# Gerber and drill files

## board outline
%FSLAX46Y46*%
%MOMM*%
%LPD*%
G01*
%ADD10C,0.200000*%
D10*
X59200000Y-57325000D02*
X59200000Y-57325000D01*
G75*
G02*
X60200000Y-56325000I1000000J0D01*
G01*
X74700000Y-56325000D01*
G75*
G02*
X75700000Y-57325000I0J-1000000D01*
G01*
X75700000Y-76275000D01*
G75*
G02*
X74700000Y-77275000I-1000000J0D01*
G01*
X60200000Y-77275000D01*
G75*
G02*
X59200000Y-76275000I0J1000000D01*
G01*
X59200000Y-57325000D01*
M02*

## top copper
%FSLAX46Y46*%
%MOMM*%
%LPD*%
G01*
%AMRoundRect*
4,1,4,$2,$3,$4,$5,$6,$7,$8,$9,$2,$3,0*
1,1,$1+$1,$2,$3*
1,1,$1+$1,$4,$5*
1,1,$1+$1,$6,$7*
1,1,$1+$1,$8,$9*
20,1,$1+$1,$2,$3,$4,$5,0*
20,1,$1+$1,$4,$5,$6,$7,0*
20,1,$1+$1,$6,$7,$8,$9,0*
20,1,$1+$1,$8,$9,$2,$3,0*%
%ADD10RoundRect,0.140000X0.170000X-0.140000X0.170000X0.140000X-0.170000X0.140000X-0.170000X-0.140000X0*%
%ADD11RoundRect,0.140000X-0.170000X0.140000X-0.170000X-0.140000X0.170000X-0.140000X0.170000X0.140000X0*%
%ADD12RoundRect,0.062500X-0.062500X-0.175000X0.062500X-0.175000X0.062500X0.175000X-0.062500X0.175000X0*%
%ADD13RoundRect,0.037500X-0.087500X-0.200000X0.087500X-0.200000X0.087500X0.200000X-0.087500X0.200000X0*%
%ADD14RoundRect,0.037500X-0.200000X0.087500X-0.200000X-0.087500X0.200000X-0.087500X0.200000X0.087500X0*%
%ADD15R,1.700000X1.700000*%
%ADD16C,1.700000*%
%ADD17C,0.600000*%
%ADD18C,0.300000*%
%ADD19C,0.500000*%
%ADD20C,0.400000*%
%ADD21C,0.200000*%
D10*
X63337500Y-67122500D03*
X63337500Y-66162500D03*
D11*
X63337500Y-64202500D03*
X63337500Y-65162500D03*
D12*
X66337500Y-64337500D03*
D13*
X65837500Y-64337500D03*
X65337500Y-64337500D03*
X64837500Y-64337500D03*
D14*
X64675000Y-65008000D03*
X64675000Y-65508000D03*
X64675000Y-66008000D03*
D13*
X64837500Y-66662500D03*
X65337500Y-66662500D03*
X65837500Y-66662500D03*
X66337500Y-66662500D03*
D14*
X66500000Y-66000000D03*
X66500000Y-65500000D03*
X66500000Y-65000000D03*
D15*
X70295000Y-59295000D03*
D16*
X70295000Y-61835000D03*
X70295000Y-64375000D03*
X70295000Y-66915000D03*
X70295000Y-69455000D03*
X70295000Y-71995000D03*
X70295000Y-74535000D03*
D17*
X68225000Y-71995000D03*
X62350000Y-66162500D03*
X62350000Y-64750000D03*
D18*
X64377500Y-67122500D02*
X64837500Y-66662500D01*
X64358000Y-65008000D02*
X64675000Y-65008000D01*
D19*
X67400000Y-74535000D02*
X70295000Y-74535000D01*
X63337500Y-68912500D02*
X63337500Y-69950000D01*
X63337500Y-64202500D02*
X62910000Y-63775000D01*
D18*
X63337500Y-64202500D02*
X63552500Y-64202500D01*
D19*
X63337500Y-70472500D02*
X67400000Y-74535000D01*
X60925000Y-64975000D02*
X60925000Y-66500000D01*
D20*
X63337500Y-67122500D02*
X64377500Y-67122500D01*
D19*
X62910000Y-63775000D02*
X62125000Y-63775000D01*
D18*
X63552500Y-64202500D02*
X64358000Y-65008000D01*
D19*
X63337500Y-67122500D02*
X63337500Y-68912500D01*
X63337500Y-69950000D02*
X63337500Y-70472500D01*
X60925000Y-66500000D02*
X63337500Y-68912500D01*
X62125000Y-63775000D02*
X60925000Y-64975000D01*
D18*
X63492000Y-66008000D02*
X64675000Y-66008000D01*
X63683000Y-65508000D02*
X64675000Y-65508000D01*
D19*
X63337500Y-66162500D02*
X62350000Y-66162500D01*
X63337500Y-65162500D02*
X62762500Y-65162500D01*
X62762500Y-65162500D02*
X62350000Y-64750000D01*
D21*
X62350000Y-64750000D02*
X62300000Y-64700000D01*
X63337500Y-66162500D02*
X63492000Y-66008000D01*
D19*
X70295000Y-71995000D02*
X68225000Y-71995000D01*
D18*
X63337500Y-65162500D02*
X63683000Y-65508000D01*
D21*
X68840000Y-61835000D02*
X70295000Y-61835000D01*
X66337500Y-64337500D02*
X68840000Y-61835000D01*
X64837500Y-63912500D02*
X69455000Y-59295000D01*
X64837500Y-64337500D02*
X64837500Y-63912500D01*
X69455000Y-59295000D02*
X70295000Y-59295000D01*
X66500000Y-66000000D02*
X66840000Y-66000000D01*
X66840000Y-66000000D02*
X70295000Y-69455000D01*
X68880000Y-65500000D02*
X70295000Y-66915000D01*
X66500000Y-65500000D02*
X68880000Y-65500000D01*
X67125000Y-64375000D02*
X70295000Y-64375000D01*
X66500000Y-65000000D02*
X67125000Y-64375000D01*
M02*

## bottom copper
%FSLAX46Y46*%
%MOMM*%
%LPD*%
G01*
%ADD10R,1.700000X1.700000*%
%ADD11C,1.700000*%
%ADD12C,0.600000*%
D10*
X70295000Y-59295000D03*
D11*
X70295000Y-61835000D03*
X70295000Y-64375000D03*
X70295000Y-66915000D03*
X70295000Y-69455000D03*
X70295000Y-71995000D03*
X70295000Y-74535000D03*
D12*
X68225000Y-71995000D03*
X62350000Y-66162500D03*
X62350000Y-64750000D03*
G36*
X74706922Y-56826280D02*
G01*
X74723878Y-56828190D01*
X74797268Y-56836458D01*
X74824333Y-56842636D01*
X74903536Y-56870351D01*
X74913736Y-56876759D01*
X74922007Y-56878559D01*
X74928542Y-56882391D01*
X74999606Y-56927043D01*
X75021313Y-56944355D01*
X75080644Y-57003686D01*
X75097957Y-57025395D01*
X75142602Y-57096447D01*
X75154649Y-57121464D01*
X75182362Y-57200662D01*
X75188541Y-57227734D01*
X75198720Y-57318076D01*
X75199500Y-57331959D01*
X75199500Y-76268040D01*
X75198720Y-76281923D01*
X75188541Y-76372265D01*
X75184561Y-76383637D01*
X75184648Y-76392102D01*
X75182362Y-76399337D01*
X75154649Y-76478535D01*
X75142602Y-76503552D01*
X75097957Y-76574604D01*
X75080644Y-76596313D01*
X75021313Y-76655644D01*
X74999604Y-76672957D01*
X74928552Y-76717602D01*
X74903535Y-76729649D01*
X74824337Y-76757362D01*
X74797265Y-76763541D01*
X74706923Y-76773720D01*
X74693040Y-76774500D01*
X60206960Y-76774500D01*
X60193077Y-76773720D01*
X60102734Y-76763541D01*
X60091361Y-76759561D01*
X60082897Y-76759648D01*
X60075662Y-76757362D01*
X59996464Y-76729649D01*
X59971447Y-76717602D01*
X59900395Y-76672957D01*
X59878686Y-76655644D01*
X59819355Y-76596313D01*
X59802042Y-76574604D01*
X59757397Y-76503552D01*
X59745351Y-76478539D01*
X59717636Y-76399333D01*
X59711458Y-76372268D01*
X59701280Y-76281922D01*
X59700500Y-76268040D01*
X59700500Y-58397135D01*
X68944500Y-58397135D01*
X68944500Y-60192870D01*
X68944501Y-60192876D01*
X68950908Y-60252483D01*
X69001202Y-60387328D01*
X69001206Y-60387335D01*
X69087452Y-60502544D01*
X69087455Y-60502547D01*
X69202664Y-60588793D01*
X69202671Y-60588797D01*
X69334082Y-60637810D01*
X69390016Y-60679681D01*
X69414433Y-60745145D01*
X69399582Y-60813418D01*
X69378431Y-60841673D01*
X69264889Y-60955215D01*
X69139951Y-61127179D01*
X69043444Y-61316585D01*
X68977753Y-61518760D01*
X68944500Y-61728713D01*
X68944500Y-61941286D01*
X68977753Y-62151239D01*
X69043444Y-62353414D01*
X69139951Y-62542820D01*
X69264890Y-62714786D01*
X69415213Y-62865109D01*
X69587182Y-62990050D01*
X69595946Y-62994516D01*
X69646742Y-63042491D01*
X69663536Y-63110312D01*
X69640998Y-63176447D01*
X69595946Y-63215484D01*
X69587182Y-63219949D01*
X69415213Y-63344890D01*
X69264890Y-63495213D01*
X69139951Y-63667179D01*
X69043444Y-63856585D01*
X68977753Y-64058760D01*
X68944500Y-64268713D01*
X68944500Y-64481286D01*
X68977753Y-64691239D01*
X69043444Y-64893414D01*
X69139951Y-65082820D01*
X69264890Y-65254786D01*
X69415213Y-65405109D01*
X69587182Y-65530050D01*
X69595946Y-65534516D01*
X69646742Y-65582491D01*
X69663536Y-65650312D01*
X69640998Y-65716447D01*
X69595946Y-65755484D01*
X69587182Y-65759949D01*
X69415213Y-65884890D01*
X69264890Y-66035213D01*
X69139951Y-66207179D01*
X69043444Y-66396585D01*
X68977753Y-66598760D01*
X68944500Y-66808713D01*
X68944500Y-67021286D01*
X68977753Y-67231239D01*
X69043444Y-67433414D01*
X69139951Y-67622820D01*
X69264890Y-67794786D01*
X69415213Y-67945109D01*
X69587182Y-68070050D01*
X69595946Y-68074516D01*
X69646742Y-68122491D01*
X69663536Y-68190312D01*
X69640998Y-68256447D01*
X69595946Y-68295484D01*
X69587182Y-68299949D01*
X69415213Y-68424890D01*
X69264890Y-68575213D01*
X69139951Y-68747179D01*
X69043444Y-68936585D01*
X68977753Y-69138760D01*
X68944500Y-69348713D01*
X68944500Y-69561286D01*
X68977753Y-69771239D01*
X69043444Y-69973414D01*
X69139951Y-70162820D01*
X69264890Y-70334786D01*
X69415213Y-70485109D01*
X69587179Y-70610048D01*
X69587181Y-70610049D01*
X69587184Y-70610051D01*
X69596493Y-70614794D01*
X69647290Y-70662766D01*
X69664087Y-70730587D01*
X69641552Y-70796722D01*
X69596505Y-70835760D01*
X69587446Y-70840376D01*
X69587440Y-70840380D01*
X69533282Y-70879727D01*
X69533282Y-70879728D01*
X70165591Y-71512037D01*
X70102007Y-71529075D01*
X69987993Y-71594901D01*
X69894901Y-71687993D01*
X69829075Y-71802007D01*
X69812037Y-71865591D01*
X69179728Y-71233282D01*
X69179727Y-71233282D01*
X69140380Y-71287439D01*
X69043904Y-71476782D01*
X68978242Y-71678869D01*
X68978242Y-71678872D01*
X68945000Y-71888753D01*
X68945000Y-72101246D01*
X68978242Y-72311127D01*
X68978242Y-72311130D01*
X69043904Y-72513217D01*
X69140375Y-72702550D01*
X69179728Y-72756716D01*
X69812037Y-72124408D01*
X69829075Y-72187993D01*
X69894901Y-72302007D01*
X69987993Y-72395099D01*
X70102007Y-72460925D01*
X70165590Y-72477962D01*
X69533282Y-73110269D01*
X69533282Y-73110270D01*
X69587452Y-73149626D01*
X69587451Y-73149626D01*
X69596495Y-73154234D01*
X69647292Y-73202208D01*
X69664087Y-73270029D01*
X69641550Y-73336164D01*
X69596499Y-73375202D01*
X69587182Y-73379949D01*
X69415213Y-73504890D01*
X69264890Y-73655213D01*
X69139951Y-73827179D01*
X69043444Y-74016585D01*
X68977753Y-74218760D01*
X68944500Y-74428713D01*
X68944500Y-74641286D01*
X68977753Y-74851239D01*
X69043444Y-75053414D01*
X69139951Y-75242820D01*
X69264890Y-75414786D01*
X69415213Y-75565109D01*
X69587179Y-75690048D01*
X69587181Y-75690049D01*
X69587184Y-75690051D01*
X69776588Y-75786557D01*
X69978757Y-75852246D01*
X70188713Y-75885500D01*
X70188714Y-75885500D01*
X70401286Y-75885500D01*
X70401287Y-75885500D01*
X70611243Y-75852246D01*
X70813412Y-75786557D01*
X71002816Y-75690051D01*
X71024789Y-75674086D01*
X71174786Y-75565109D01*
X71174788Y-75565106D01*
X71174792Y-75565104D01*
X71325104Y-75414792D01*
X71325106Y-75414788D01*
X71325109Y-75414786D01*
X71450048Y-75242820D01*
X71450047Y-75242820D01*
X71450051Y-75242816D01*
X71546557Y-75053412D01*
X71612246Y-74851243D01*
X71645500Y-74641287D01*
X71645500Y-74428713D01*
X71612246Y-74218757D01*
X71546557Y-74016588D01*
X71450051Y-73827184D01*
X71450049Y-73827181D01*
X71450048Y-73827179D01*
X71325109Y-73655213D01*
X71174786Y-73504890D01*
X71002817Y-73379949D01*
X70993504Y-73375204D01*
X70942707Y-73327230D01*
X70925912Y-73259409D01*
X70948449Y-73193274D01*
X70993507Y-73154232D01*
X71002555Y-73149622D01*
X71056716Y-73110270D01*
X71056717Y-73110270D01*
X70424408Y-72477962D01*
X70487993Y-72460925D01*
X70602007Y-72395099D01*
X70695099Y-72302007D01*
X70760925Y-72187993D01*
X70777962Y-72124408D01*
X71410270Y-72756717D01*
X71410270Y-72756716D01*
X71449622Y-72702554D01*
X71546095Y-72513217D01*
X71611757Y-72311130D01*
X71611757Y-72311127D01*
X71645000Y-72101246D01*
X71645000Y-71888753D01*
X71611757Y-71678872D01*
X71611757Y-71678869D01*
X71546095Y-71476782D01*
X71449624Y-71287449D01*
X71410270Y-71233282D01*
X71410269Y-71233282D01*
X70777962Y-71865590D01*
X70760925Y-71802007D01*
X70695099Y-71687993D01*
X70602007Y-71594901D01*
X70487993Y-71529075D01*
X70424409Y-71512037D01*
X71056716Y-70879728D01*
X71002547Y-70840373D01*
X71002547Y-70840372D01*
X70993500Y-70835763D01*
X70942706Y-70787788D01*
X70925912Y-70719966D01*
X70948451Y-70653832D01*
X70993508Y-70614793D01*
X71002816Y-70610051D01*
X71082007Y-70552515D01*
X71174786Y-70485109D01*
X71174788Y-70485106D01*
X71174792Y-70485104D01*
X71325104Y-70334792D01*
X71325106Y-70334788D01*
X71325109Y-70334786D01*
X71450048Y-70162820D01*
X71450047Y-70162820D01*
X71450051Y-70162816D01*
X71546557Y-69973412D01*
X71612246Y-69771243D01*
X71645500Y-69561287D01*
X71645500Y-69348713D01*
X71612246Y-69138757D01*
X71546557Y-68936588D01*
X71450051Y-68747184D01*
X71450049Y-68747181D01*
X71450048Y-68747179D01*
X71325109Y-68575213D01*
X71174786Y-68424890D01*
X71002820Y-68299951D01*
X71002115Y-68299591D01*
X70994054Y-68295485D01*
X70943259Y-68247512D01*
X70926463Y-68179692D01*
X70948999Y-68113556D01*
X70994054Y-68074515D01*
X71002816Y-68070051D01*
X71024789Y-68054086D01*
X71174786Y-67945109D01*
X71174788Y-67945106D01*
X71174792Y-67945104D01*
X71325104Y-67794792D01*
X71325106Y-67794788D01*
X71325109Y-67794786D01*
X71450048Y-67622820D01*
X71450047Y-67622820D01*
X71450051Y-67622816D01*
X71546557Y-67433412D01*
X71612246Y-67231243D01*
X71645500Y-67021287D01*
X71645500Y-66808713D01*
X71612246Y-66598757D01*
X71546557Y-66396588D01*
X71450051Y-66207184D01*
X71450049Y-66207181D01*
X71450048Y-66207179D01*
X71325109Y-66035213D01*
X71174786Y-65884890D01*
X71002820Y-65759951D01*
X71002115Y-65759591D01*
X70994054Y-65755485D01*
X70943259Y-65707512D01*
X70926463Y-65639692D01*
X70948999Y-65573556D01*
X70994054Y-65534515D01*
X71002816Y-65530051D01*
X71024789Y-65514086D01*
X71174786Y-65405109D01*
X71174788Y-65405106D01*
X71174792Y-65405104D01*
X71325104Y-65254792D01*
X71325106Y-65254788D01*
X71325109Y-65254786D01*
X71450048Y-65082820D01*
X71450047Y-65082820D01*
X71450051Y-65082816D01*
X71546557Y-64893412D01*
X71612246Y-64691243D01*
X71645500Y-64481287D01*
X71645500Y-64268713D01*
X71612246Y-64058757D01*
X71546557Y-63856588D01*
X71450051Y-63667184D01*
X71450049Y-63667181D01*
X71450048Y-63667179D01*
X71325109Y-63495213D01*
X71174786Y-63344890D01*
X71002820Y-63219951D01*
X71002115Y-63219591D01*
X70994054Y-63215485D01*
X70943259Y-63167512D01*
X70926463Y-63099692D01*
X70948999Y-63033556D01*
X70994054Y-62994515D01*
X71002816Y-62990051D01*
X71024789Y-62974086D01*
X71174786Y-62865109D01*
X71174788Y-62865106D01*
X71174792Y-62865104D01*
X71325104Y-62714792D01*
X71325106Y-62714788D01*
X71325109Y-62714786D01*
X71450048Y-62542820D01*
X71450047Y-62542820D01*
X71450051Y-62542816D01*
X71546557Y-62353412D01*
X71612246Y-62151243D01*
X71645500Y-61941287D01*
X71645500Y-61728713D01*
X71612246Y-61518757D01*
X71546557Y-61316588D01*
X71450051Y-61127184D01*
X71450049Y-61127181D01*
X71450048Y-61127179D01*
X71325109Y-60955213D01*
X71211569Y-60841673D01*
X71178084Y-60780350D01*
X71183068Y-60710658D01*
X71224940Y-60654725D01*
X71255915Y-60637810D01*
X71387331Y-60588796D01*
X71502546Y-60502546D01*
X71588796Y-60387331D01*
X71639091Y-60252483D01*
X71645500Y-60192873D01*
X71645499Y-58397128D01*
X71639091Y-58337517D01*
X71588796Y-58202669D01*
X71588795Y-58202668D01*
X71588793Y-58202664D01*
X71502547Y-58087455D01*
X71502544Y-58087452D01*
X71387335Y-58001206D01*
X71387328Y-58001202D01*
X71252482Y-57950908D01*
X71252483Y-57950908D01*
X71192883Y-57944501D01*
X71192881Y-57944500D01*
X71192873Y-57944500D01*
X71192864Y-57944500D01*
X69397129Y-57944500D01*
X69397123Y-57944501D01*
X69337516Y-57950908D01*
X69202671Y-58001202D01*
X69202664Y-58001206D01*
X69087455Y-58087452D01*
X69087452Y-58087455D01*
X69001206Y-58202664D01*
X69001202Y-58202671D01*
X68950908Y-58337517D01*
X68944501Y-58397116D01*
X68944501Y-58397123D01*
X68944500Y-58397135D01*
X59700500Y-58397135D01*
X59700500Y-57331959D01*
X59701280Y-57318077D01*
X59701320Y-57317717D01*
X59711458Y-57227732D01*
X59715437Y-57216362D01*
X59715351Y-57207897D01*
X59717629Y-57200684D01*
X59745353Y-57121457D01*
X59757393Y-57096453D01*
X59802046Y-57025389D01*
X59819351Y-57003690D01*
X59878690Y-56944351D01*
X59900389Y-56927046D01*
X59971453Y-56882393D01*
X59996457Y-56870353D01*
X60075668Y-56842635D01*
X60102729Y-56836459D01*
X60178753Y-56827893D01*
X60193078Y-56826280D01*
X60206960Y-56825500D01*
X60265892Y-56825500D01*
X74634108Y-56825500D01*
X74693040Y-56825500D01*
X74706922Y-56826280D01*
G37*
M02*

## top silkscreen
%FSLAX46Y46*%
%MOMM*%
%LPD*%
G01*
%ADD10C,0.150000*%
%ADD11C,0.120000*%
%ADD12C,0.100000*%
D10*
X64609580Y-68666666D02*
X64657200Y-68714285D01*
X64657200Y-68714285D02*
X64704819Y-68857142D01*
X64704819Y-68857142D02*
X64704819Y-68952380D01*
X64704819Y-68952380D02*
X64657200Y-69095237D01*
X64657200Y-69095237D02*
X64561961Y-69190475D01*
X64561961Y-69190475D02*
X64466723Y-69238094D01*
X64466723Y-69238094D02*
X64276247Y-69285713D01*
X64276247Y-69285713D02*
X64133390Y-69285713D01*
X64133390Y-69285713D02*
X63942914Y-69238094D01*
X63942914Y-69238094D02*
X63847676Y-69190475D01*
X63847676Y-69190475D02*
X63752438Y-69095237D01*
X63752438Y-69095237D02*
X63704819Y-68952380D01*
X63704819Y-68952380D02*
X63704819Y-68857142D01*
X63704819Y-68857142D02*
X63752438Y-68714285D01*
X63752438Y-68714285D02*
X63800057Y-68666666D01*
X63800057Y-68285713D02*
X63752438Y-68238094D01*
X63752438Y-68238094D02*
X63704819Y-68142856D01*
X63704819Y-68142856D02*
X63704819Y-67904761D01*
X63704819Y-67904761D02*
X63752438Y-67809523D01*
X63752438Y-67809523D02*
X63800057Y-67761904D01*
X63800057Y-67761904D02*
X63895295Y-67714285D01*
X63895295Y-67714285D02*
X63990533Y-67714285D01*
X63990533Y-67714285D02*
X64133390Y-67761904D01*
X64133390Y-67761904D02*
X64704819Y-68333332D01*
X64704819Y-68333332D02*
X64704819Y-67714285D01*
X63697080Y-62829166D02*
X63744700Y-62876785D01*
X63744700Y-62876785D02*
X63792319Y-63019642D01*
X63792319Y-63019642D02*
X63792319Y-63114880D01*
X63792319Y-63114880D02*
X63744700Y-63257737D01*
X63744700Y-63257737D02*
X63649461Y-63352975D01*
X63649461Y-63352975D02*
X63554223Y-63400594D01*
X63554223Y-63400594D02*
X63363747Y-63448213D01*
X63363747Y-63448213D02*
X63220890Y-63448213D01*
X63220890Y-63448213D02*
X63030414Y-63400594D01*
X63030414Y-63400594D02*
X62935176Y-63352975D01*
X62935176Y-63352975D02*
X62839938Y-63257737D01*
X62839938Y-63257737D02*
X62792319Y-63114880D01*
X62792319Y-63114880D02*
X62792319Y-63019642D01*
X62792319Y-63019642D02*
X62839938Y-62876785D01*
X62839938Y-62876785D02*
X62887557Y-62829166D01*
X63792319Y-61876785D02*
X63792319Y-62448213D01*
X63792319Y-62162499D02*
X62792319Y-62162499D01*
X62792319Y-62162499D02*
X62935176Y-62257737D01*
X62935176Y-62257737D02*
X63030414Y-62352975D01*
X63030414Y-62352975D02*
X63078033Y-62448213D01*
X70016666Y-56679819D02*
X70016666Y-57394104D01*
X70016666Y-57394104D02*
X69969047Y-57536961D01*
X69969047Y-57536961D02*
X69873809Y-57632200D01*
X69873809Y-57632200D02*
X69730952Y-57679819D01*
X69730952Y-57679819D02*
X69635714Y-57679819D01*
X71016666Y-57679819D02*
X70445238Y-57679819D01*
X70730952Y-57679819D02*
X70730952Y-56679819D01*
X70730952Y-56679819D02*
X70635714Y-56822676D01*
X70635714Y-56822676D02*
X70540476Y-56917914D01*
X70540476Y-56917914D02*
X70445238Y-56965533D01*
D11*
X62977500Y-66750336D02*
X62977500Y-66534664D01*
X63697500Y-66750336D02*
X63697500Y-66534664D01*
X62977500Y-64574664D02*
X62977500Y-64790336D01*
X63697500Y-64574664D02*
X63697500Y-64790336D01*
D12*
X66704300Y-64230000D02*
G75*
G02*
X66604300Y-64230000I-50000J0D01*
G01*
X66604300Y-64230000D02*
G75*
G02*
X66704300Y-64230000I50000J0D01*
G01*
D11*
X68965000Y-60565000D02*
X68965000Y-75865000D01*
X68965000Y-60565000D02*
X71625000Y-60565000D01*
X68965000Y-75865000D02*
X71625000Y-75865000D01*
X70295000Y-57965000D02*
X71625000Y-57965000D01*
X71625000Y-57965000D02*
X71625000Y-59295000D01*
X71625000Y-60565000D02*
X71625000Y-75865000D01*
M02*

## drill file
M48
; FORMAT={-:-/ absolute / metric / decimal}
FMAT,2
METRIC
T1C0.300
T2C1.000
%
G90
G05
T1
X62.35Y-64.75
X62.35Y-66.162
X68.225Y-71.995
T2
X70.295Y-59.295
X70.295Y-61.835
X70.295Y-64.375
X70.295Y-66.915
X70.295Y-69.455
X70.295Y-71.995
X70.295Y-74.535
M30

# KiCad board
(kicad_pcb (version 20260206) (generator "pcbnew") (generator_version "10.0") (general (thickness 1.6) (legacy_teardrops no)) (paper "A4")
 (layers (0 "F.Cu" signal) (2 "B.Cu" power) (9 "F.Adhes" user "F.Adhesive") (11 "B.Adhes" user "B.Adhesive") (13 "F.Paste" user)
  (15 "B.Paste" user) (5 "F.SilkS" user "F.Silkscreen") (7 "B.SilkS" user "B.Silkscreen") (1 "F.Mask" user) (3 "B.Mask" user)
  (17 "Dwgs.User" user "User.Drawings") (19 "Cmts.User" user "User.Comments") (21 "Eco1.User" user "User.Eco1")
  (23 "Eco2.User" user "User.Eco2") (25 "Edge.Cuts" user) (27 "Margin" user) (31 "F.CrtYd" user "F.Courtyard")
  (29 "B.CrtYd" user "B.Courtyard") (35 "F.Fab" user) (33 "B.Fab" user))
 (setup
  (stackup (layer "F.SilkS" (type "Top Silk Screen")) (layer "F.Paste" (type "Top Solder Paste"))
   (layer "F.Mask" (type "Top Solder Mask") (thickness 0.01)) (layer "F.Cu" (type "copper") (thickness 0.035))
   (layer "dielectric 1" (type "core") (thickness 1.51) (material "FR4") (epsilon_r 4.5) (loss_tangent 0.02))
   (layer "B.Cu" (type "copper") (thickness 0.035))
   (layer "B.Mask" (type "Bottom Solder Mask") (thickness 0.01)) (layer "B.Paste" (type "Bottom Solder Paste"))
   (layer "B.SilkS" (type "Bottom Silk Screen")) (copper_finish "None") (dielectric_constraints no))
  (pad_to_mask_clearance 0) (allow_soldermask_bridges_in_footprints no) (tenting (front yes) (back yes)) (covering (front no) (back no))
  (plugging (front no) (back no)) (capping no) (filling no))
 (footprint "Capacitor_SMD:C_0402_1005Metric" (layer "F.Cu") (at 63.3375 66.6425 90)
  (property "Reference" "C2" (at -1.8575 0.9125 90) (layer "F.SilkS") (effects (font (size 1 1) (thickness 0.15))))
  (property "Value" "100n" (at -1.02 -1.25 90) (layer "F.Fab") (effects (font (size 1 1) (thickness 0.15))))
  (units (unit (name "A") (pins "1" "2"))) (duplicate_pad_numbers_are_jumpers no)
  (fp_line (start -0.107836 -0.36) (end 0.107836 -0.36) (stroke (width 0.12) (type solid)) (layer "F.SilkS"))
  (fp_line (start -0.107836 0.36) (end 0.107836 0.36) (stroke (width 0.12) (type solid)) (layer "F.SilkS"))
  (pad "1" smd roundrect (at -0.48 0 90) (size 0.56 0.62) (layers "F.Cu" "F.Mask" "F.Paste") (roundrect_rratio 0.25) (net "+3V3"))
  (pad "2" smd roundrect (at 0.48 0 90) (size 0.56 0.62) (layers "F.Cu" "F.Mask" "F.Paste") (roundrect_rratio 0.25) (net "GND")))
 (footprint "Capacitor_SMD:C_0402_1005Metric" (layer "F.Cu") (at 63.3375 64.6825 -90)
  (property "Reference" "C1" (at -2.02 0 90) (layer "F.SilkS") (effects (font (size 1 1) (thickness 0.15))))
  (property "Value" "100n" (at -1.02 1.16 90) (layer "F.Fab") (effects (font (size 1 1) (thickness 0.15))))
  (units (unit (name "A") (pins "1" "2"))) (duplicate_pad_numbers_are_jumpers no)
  (fp_line (start -0.107836 0.36) (end 0.107836 0.36) (stroke (width 0.12) (type solid)) (layer "F.SilkS"))
  (fp_line (start -0.107836 -0.36) (end 0.107836 -0.36) (stroke (width 0.12) (type solid)) (layer "F.SilkS"))
  (pad "1" smd roundrect (at -0.48 0 270) (size 0.56 0.62) (layers "F.Cu" "F.Mask" "F.Paste") (roundrect_rratio 0.25) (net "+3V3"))
  (pad "2" smd roundrect (at 0.48 0 270) (size 0.56 0.62) (layers "F.Cu" "F.Mask" "F.Paste") (roundrect_rratio 0.25) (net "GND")))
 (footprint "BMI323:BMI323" (layer "F.Cu") (at 65.5875 65.5 -90)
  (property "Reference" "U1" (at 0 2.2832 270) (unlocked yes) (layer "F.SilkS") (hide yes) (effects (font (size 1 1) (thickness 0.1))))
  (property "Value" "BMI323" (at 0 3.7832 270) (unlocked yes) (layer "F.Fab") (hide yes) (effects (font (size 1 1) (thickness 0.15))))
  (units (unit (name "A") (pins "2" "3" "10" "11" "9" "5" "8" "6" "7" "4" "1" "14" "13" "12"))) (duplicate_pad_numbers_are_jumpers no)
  (fp_circle (center -1.27 -1.0668) (end -1.17 -1.0668) (stroke (width 0) (type solid)) (fill yes) (layer "F.SilkS"))
  (pad "1" smd roundrect (at -1.1625 -0.75) (size 0.25 0.475) (layers "F.Cu" "F.Mask") (roundrect_rratio 0.25) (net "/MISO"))
  (pad "2" smd roundrect (at -1.1625 -0.25) (size 0.25 0.475) (layers "F.Cu" "F.Mask") (roundrect_rratio 0.15)
   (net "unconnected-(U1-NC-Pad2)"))
  (pad "3" smd roundrect (at -1.1625 0.25) (size 0.25 0.475) (layers "F.Cu" "F.Mask") (roundrect_rratio 0.15)
   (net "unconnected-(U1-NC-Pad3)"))
  (pad "4" smd roundrect (at -1.1625 0.75) (size 0.25 0.475) (layers "F.Cu" "F.Mask") (roundrect_rratio 0.15) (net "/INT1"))
  (pad "5" smd roundrect (at -0.492 0.9125 270) (size 0.25 0.475) (layers "F.Cu" "F.Mask") (roundrect_rratio 0.15) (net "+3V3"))
  (pad "6" smd roundrect (at 0.008 0.9125 270) (size 0.25 0.475) (layers "F.Cu" "F.Mask") (roundrect_rratio 0.15) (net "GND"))
  (pad "7" smd roundrect (at 0.508 0.9125 270) (size 0.25 0.475) (layers "F.Cu" "F.Mask") (roundrect_rratio 0.15) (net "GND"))
  (pad "8" smd roundrect (at 1.1625 0.75) (size 0.25 0.475) (layers "F.Cu" "F.Mask") (roundrect_rratio 0.15) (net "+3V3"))
  (pad "9" smd roundrect (at 1.1625 0.25) (size 0.25 0.475) (layers "F.Cu" "F.Mask") (roundrect_rratio 0.15)
   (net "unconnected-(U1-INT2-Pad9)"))
  (pad "10" smd roundrect (at 1.1625 -0.25) (size 0.25 0.475) (layers "F.Cu" "F.Mask") (roundrect_rratio 0.15)
   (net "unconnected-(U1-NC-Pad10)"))
  (pad "11" smd roundrect (at 1.1625 -0.75) (size 0.25 0.475) (layers "F.Cu" "F.Mask") (roundrect_rratio 0.15)
   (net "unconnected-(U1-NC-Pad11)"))
  (pad "12" smd roundrect (at 0.5 -0.9125 270) (size 0.25 0.475) (layers "F.Cu" "F.Mask") (roundrect_rratio 0.15) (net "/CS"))
  (pad "13" smd roundrect (at 0 -0.9125 270) (size 0.25 0.475) (layers "F.Cu" "F.Mask") (roundrect_rratio 0.15) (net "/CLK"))
  (pad "14" smd roundrect (at -0.5 -0.9125 270) (size 0.25 0.475) (layers "F.Cu" "F.Mask") (roundrect_rratio 0.15) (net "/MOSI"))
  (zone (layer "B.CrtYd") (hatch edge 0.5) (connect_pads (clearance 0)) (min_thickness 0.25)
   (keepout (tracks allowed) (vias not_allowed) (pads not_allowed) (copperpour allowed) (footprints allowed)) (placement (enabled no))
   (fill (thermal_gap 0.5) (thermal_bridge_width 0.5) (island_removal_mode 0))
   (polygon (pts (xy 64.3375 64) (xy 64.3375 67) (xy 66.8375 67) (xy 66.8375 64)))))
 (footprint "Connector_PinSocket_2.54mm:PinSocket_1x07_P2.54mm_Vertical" (layer "F.Cu") (at 70.295 59.295)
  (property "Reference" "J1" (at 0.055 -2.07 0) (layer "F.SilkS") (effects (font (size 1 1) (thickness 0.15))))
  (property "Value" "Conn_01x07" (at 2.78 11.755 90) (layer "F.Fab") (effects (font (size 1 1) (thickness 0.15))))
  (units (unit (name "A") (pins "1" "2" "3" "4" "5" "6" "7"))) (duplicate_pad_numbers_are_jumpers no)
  (fp_line (start -1.33 1.27) (end -1.33 16.57) (stroke (width 0.12) (type solid)) (layer "F.SilkS"))
  (fp_line (start -1.33 1.27) (end 1.33 1.27) (stroke (width 0.12) (type solid)) (layer "F.SilkS"))
  (fp_line (start -1.33 16.57) (end 1.33 16.57) (stroke (width 0.12) (type solid)) (layer "F.SilkS"))
  (fp_line (start 0 -1.33) (end 1.33 -1.33) (stroke (width 0.12) (type solid)) (layer "F.SilkS"))
  (fp_line (start 1.33 -1.33) (end 1.33 0) (stroke (width 0.12) (type solid)) (layer "F.SilkS"))
  (fp_line (start 1.33 1.27) (end 1.33 16.57) (stroke (width 0.12) (type solid)) (layer "F.SilkS"))
  (pad "1" thru_hole rect (at 0 0) (size 1.7 1.7) (drill 1) (layers "*.Cu" "*.Mask") (remove_unused_layers no) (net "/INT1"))
  (pad "2" thru_hole circle (at 0 2.54) (size 1.7 1.7) (drill 1) (layers "*.Cu" "*.Mask") (remove_unused_layers no) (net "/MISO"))
  (pad "3" thru_hole circle (at 0 5.08) (size 1.7 1.7) (drill 1) (layers "*.Cu" "*.Mask") (remove_unused_layers no) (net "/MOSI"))
  (pad "4" thru_hole circle (at 0 7.62) (size 1.7 1.7) (drill 1) (layers "*.Cu" "*.Mask") (remove_unused_layers no) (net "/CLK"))
  (pad "5" thru_hole circle (at 0 10.16) (size 1.7 1.7) (drill 1) (layers "*.Cu" "*.Mask") (remove_unused_layers no) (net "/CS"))
  (pad "6" thru_hole circle (at 0 12.7) (size 1.7 1.7) (drill 1) (layers "*.Cu" "*.Mask") (remove_unused_layers no) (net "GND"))
  (pad "7" thru_hole circle (at 0 15.24) (size 1.7 1.7) (drill 1) (layers "*.Cu" "*.Mask") (remove_unused_layers no) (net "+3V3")))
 (gr_rect (start 59.2 56.325) (end 75.7 77.275) (radius 1) (stroke (width 0.2) (type solid)) (fill no) (layer "Edge.Cuts"))
 (segment (start 64.3775 67.1225) (end 64.8375 66.6625) (width 0.3) (layer "F.Cu") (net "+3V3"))
 (segment (start 64.358 65.008) (end 64.675 65.008) (width 0.3) (layer "F.Cu") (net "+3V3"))
 (segment (start 67.4 74.535) (end 70.295 74.535) (width 0.5) (layer "F.Cu") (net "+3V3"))
 (segment (start 63.3375 68.9125) (end 63.3375 69.95) (width 0.5) (layer "F.Cu") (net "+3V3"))
 (segment (start 63.3375 64.2025) (end 62.91 63.775) (width 0.5) (layer "F.Cu") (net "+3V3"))
 (segment (start 63.3375 64.2025) (end 63.5525 64.2025) (width 0.3) (layer "F.Cu") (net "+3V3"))
 (segment (start 63.3375 70.4725) (end 67.4 74.535) (width 0.5) (layer "F.Cu") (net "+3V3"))
 (segment (start 60.925 64.975) (end 60.925 66.5) (width 0.5) (layer "F.Cu") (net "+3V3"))
 (segment (start 63.3375 67.1225) (end 64.3775 67.1225) (width 0.4) (layer "F.Cu") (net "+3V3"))
 (segment (start 62.91 63.775) (end 62.125 63.775) (width 0.5) (layer "F.Cu") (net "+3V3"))
 (segment (start 63.5525 64.2025) (end 64.358 65.008) (width 0.3) (layer "F.Cu") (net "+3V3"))
 (segment (start 63.3375 67.1225) (end 63.3375 68.9125) (width 0.5) (layer "F.Cu") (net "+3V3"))
 (segment (start 63.3375 69.95) (end 63.3375 70.4725) (width 0.5) (layer "F.Cu") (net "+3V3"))
 (segment (start 60.925 66.5) (end 63.3375 68.9125) (width 0.5) (layer "F.Cu") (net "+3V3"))
 (segment (start 62.125 63.775) (end 60.925 64.975) (width 0.5) (layer "F.Cu") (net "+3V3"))
 (segment (start 63.492 66.008) (end 64.675 66.008) (width 0.3) (layer "F.Cu") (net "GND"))
 (segment (start 63.683 65.508) (end 64.675 65.508) (width 0.3) (layer "F.Cu") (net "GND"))
 (segment (start 63.3375 66.1625) (end 62.35 66.1625) (width 0.5) (layer "F.Cu") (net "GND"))
 (segment (start 63.3375 65.1625) (end 62.7625 65.1625) (width 0.5) (layer "F.Cu") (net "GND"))
 (segment (start 62.7625 65.1625) (end 62.35 64.75) (width 0.5) (layer "F.Cu") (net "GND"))
 (segment (start 62.35 64.75) (end 62.3 64.7) (width 0.2) (layer "F.Cu") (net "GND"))
 (segment (start 63.3375 66.1625) (end 63.492 66.008) (width 0.2) (layer "F.Cu") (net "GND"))
 (segment (start 70.295 71.995) (end 68.225 71.995) (width 0.5) (layer "F.Cu") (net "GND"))
 (segment (start 63.3375 65.1625) (end 63.683 65.508) (width 0.3) (layer "F.Cu") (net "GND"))
 (via (at 68.225 71.995) (size 0.6) (drill 0.3) (layers "F.Cu" "B.Cu") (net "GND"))
 (via (at 62.35 66.1625) (size 0.6) (drill 0.3) (layers "F.Cu" "B.Cu") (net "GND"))
 (via (at 62.35 64.75) (size 0.6) (drill 0.3) (layers "F.Cu" "B.Cu") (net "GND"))
 (segment (start 68.84 61.835) (end 70.295 61.835) (width 0.2) (layer "F.Cu") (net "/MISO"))
 (segment (start 66.3375 64.3375) (end 68.84 61.835) (width 0.2) (layer "F.Cu") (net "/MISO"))
 (segment (start 64.8375 63.9125) (end 69.455 59.295) (width 0.2) (layer "F.Cu") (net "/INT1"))
 (segment (start 64.8375 64.3375) (end 64.8375 63.9125) (width 0.2) (layer "F.Cu") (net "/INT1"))
 (segment (start 69.455 59.295) (end 70.295 59.295) (width 0.2) (layer "F.Cu") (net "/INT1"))
 (segment (start 66.5 66) (end 66.84 66) (width 0.2) (layer "F.Cu") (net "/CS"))
 (segment (start 66.84 66) (end 70.295 69.455) (width 0.2) (layer "F.Cu") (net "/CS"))
 (segment (start 68.88 65.5) (end 70.295 66.915) (width 0.2) (layer "F.Cu") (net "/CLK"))
 (segment (start 66.5 65.5) (end 68.88 65.5) (width 0.2) (layer "F.Cu") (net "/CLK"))
 (segment (start 67.125 64.375) (end 70.295 64.375) (width 0.2) (layer "F.Cu") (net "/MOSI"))
 (segment (start 66.5 65) (end 67.125 64.375) (width 0.2) (layer "F.Cu") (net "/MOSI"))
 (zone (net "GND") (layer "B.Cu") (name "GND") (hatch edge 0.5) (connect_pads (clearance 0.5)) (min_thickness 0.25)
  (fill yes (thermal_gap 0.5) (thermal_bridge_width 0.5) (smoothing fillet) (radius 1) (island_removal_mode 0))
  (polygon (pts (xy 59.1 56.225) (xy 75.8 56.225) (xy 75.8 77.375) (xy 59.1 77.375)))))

